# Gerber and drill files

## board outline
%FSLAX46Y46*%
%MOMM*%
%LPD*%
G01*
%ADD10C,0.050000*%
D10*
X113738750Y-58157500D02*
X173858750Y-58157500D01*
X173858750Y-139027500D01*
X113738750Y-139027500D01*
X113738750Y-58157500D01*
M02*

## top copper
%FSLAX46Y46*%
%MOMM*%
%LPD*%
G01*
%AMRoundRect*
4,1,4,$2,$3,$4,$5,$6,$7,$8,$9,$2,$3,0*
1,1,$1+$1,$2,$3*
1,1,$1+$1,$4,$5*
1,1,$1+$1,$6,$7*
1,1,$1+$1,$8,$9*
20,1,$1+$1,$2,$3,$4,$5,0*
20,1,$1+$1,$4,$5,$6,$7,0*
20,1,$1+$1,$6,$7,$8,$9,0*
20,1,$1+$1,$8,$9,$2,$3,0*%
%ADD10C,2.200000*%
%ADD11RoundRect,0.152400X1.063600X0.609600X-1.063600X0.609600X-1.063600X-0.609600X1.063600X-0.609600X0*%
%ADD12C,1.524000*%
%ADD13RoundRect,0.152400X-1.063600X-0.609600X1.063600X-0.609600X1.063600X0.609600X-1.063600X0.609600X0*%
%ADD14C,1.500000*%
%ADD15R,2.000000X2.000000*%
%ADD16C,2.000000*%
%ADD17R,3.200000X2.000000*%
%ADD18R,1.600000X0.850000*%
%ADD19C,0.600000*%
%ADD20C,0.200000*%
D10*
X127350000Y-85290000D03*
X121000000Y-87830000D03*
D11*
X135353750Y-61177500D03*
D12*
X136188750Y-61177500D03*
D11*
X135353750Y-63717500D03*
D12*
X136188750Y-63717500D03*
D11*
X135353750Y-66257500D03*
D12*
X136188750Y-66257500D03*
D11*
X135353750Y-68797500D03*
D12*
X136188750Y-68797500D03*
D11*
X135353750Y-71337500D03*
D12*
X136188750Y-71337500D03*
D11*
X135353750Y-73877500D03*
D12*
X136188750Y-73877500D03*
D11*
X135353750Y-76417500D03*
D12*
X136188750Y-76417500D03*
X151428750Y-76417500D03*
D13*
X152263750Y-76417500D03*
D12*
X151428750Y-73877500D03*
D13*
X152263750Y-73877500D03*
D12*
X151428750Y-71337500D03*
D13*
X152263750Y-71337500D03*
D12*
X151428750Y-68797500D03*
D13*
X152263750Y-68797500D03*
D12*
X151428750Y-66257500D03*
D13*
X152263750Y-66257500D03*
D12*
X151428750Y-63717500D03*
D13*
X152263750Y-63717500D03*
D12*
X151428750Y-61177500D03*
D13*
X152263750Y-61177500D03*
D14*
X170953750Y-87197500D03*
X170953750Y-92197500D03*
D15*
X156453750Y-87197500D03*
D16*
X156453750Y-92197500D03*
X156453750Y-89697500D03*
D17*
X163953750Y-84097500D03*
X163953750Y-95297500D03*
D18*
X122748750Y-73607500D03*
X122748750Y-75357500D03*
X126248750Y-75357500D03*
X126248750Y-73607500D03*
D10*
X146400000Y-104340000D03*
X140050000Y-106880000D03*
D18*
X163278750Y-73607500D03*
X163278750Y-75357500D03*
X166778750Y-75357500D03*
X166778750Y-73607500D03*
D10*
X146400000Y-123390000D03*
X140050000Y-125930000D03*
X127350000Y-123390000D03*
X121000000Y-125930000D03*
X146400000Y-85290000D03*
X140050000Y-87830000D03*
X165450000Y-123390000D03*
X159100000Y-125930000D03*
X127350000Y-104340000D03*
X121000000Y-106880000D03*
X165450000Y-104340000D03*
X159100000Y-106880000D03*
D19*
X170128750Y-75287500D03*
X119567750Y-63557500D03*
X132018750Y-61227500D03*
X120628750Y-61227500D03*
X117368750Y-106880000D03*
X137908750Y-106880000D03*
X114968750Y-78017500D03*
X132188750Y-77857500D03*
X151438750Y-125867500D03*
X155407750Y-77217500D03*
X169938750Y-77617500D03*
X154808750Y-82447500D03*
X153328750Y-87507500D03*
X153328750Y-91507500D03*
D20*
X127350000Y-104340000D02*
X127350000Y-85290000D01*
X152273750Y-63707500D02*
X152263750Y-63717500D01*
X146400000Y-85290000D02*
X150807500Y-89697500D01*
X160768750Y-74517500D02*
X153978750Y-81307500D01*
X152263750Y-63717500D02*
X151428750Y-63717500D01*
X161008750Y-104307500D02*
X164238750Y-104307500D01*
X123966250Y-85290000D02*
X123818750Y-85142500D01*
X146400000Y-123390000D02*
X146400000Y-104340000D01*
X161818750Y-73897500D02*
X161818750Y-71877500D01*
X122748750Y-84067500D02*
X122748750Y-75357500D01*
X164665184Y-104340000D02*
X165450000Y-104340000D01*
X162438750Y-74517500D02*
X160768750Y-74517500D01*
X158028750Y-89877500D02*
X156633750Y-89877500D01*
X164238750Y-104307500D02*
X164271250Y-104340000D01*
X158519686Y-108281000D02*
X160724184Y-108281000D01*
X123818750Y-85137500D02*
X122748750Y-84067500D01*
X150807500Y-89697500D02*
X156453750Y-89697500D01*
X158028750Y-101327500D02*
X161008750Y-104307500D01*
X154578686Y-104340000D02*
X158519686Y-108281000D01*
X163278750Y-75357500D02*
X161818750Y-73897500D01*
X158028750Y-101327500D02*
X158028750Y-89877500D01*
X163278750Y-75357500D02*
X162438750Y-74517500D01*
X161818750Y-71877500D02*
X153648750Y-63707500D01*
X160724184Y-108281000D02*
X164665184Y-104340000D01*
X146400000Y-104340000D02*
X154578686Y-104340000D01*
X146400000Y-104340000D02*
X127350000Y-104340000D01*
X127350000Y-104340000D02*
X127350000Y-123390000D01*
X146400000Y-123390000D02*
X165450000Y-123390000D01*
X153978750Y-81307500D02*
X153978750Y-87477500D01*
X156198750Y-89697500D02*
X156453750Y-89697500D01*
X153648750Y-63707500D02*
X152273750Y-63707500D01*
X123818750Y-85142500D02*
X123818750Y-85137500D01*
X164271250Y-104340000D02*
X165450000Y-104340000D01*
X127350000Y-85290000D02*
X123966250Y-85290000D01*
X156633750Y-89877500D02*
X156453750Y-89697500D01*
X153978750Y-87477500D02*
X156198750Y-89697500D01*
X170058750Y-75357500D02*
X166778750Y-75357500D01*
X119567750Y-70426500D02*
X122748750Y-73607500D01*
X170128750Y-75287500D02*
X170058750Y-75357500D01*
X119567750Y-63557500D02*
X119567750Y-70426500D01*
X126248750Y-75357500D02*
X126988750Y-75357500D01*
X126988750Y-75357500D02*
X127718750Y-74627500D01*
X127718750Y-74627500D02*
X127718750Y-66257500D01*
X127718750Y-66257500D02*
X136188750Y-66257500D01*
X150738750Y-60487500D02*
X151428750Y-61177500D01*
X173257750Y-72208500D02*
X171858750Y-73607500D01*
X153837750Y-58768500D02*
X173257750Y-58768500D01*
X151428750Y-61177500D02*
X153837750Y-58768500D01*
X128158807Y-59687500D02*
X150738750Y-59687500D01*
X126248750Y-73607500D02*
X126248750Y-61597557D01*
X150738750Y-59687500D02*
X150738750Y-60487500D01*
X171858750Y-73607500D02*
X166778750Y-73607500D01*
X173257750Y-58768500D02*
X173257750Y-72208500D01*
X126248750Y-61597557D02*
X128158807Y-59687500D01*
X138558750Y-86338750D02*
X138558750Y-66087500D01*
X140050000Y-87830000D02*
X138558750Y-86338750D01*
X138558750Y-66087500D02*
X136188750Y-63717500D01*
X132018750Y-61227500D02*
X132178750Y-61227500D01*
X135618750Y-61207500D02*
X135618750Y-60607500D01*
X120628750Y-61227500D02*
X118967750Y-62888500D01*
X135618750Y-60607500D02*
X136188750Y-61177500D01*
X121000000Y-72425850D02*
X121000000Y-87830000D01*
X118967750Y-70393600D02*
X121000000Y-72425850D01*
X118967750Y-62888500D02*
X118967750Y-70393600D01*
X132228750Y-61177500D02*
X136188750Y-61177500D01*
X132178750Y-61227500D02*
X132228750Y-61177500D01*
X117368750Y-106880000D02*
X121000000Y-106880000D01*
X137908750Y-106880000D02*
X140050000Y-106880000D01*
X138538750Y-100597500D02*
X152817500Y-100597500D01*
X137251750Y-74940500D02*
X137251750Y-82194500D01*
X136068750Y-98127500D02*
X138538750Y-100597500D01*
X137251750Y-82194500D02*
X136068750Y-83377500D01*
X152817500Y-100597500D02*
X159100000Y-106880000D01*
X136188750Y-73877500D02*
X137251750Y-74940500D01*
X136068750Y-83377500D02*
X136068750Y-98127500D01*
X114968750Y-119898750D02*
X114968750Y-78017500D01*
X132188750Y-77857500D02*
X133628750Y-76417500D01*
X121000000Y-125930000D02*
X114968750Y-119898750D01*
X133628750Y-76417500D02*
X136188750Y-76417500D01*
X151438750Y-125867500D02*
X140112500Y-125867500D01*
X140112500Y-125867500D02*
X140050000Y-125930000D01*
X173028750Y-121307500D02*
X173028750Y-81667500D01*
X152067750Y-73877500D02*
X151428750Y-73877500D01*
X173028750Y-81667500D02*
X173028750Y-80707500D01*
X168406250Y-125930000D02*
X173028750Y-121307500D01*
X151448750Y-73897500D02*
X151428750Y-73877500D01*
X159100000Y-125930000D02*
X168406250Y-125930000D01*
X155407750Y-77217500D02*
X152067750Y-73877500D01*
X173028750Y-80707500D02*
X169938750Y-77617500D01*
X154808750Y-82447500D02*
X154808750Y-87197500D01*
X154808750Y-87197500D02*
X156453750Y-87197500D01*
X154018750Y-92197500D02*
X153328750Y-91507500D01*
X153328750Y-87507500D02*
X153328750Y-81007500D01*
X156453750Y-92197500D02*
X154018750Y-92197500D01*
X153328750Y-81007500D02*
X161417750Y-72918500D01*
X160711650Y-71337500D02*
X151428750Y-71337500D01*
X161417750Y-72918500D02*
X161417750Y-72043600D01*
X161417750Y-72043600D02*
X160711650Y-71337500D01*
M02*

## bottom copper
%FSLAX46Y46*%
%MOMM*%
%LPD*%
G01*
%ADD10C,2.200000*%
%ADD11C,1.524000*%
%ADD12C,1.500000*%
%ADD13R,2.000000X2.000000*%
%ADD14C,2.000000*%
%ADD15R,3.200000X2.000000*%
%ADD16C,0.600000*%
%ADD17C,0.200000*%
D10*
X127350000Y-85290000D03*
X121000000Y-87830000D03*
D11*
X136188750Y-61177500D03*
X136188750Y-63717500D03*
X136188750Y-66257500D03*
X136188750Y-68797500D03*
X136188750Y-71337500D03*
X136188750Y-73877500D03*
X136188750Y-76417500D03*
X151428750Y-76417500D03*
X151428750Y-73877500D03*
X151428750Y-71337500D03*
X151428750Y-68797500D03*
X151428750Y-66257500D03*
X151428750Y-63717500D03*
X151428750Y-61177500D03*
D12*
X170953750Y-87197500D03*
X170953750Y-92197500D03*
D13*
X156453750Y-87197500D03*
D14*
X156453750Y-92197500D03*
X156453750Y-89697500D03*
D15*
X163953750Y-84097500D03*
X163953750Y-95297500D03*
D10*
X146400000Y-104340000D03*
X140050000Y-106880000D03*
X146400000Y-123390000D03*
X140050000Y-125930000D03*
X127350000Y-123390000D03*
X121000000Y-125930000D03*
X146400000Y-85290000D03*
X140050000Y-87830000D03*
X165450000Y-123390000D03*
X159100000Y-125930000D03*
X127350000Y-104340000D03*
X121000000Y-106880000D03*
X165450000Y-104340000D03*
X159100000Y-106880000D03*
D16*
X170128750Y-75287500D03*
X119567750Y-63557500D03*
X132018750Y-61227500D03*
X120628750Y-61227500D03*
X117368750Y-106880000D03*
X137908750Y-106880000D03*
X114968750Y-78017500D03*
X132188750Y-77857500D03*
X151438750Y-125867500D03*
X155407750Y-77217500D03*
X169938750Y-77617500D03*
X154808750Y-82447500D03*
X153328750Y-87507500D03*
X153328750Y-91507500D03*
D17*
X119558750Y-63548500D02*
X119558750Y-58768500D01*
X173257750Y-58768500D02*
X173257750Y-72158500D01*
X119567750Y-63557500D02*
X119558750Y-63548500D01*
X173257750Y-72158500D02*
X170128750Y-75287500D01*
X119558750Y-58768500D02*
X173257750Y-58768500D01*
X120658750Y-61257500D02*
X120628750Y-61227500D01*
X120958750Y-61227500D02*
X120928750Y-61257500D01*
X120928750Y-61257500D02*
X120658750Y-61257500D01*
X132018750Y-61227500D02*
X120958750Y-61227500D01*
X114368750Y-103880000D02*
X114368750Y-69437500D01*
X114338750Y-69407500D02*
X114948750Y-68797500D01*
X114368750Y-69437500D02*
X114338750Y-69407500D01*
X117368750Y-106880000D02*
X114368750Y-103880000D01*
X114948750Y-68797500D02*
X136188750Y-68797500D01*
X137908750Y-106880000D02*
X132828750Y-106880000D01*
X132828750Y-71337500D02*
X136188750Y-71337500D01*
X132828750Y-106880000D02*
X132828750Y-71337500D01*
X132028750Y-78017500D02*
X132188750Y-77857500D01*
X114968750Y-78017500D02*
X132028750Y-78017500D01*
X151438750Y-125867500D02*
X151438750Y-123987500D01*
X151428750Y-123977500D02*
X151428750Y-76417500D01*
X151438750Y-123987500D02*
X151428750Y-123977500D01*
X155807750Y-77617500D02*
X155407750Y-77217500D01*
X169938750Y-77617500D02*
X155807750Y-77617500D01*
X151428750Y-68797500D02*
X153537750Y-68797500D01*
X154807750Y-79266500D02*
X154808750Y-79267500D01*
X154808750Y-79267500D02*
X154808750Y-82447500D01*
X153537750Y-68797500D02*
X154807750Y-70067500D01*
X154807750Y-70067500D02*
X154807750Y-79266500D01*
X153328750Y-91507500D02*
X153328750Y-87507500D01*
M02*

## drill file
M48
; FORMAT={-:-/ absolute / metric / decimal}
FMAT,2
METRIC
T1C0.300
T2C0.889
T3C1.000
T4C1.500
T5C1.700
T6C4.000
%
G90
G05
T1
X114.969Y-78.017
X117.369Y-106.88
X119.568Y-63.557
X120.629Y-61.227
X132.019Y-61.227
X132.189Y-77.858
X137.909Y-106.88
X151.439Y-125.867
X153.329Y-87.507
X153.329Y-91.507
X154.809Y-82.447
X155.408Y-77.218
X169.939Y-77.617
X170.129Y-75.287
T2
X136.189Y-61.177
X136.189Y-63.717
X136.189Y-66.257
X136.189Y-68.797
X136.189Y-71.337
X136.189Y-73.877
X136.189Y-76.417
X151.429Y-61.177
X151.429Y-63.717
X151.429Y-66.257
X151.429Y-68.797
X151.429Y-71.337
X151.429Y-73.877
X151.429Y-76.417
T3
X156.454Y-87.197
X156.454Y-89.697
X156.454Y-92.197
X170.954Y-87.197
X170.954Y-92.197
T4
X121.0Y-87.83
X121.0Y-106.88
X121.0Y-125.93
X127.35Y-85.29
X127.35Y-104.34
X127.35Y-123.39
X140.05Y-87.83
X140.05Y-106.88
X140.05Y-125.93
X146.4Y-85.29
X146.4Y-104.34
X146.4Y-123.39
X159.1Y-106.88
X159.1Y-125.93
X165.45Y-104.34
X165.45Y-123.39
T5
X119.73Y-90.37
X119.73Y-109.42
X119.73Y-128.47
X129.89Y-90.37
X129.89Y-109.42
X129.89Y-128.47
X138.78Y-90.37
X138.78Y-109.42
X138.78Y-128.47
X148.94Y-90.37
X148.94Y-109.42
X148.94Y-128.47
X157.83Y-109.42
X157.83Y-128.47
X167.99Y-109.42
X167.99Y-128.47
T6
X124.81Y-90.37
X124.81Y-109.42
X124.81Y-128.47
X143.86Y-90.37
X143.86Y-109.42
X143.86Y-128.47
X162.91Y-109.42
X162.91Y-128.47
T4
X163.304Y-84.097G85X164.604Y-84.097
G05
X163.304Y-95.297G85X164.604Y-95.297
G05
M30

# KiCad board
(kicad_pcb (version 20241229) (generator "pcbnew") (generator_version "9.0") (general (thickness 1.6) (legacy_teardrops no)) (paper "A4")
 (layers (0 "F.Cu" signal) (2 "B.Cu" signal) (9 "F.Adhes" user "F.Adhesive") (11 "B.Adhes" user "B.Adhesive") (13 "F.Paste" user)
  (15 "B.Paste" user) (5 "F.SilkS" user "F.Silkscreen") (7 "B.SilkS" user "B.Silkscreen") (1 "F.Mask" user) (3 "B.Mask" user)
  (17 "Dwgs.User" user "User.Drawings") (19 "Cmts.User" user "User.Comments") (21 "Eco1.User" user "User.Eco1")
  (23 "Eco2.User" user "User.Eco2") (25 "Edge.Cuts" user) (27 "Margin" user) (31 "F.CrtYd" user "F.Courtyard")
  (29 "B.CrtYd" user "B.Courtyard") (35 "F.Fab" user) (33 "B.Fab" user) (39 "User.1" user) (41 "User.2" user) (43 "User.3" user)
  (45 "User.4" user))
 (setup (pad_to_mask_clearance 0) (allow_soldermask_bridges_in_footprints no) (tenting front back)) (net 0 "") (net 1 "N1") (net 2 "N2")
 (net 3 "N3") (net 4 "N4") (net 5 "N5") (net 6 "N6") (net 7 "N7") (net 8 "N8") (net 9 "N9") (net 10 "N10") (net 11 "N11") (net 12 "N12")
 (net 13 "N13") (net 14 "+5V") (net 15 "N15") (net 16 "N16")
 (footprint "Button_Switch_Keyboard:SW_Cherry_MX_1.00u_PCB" (layer "F.Cu") (at 127.35 85.29)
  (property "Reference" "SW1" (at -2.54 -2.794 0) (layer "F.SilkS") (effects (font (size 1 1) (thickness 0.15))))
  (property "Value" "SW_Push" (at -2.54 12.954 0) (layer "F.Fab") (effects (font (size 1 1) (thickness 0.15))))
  (pad "" np_thru_hole circle (at -7.62 5.08) (size 1.7 1.7) (drill 1.7) (layers "*.Cu" "*.Mask"))
  (pad "" np_thru_hole circle (at -2.54 5.08) (size 4 4) (drill 4) (layers "*.Cu" "*.Mask"))
  (pad "" np_thru_hole circle (at 2.54 5.08) (size 1.7 1.7) (drill 1.7) (layers "*.Cu" "*.Mask"))
  (pad "1" thru_hole circle (at 0 0) (size 2.2 2.2) (drill 1.5) (layers "*.Cu" "*.Mask") (remove_unused_layers no) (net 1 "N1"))
  (pad "2" thru_hole circle (at -6.35 2.54) (size 2.2 2.2) (drill 1.5) (layers "*.Cu" "*.Mask") (remove_unused_layers no) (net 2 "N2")))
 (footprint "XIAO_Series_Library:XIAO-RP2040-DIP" (layer "F.Cu") (at 143.80875 68.7975)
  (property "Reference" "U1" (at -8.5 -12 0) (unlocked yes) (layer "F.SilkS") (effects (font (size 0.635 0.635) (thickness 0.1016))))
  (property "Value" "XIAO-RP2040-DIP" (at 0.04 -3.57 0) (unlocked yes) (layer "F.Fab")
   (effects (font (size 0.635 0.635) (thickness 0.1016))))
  (pad "1" smd roundrect (at -8.455 -7.62 180) (size 2.432 1.524) (layers "F.Cu" "F.Mask") (roundrect_rratio 0.1) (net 2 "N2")
   (thermal_bridge_angle 45))
  (pad "1" thru_hole circle (at -7.62 -7.62 180) (size 1.524 1.524) (drill 0.889) (layers "*.Cu" "*.Mask") (remove_unused_layers no)
   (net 2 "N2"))
  (pad "2" smd roundrect (at -8.455 -5.08 180) (size 2.432 1.524) (layers "F.Cu" "F.Mask") (roundrect_rratio 0.1) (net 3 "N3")
   (thermal_bridge_angle 45))
  (pad "2" thru_hole circle (at -7.62 -5.08 180) (size 1.524 1.524) (drill 0.889) (layers "*.Cu" "*.Mask") (remove_unused_layers no)
   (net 3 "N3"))
  (pad "3" smd roundrect (at -8.455 -2.54 180) (size 2.432 1.524) (layers "F.Cu" "F.Mask") (roundrect_rratio 0.1) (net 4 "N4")
   (thermal_bridge_angle 45))
  (pad "3" thru_hole circle (at -7.62 -2.54 180) (size 1.524 1.524) (drill 0.889) (layers "*.Cu" "*.Mask") (remove_unused_layers no)
   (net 4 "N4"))
  (pad "4" smd roundrect (at -8.455 0 180) (size 2.432 1.524) (layers "F.Cu" "F.Mask") (roundrect_rratio 0.1) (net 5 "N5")
   (thermal_bridge_angle 45))
  (pad "4" thru_hole circle (at -7.62 0 180) (size 1.524 1.524) (drill 0.889) (layers "*.Cu" "*.Mask") (remove_unused_layers no)
   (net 5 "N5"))
  (pad "5" smd roundrect (at -8.455 2.54 180) (size 2.432 1.524) (layers "F.Cu" "F.Mask") (roundrect_rratio 0.1) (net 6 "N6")
   (thermal_bridge_angle 45))
  (pad "5" thru_hole circle (at -7.62 2.54 180) (size 1.524 1.524) (drill 0.889) (layers "*.Cu" "*.Mask") (remove_unused_layers no)
   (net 6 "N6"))
  (pad "6" smd roundrect (at -8.455 5.08 180) (size 2.432 1.524) (layers "F.Cu" "F.Mask") (roundrect_rratio 0.1) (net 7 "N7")
   (thermal_bridge_angle 45))
  (pad "6" thru_hole circle (at -7.62 5.08 180) (size 1.524 1.524) (drill 0.889) (layers "*.Cu" "*.Mask") (remove_unused_layers no)
   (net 7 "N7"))
  (pad "7" smd roundrect (at -8.455 7.62 180) (size 2.432 1.524) (layers "F.Cu" "F.Mask") (roundrect_rratio 0.1) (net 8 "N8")
   (thermal_bridge_angle 45))
  (pad "7" thru_hole circle (at -7.62 7.62 180) (size 1.524 1.524) (drill 0.889) (layers "*.Cu" "*.Mask") (remove_unused_layers no)
   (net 8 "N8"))
  (pad "8" thru_hole circle (at 7.62 7.62) (size 1.524 1.524) (drill 0.889) (layers "*.Cu" "*.Mask") (remove_unused_layers no) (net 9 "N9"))
  (pad "8" smd roundrect (at 8.455 7.62) (size 2.432 1.524) (layers "F.Cu" "F.Mask") (roundrect_rratio 0.1) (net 9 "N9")
   (thermal_bridge_angle 45))
  (pad "9" thru_hole circle (at 7.62 5.08) (size 1.524 1.524) (drill 0.889) (layers "*.Cu" "*.Mask") (remove_unused_layers no)
   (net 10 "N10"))
  (pad "9" smd roundrect (at 8.455 5.08) (size 2.432 1.524) (layers "F.Cu" "F.Mask") (roundrect_rratio 0.1) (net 10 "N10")
   (thermal_bridge_angle 45))
  (pad "10" thru_hole circle (at 7.62 2.54) (size 1.524 1.524) (drill 0.889) (layers "*.Cu" "*.Mask") (remove_unused_layers no)
   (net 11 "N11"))
  (pad "10" smd roundrect (at 8.455 2.54) (size 2.432 1.524) (layers "F.Cu" "F.Mask") (roundrect_rratio 0.1) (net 11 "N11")
   (thermal_bridge_angle 45))
  (pad "11" thru_hole circle (at 7.62 0) (size 1.524 1.524) (drill 0.889) (layers "*.Cu" "*.Mask") (remove_unused_layers no) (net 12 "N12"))
  (pad "11" smd roundrect (at 8.455 0) (size 2.432 1.524) (layers "F.Cu" "F.Mask") (roundrect_rratio 0.1) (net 12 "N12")
   (thermal_bridge_angle 45))
  (pad "12" thru_hole circle (at 7.62 -2.54) (size 1.524 1.524) (drill 0.889) (layers "*.Cu" "*.Mask") (remove_unused_layers no)
   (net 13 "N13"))
  (pad "12" smd roundrect (at 8.455 -2.54) (size 2.432 1.524) (layers "F.Cu" "F.Mask") (roundrect_rratio 0.1) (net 13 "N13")
   (thermal_bridge_angle 45))
  (pad "13" thru_hole circle (at 7.62 -5.08) (size 1.524 1.524) (drill 0.889) (layers "*.Cu" "*.Mask") (remove_unused_layers no)
   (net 1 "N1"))
  (pad "13" smd roundrect (at 8.455 -5.08) (size 2.432 1.524) (layers "F.Cu" "F.Mask") (roundrect_rratio 0.1) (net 1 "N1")
   (thermal_bridge_angle 45))
  (pad "14" thru_hole circle (at 7.62 -7.62) (size 1.524 1.524) (drill 0.889) (layers "*.Cu" "*.Mask") (remove_unused_layers no)
   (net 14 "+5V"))
  (pad "14" smd roundrect (at 8.455 -7.62) (size 2.432 1.524) (layers "F.Cu" "F.Mask") (roundrect_rratio 0.1) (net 14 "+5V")
   (thermal_bridge_angle 45)))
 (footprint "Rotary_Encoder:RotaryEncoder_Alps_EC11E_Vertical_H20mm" (layer "F.Cu") (at 156.45375 87.1975)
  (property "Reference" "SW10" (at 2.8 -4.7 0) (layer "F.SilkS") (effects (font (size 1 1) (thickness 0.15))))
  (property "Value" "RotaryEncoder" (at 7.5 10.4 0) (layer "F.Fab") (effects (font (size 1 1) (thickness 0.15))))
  (pad "" thru_hole circle (at 14.5 0) (size 1.5 1.5) (drill 1) (layers "*.Cu" "*.Mask") (remove_unused_layers no))
  (pad "" thru_hole circle (at 14.5 5) (size 1.5 1.5) (drill 1) (layers "*.Cu" "*.Mask") (remove_unused_layers no))
  (pad "A" thru_hole rect (at 0 0) (size 2 2) (drill 1) (layers "*.Cu" "*.Mask") (remove_unused_layers no) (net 12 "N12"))
  (pad "B" thru_hole circle (at 0 5) (size 2 2) (drill 1) (layers "*.Cu" "*.Mask") (remove_unused_layers no) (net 11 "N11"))
  (pad "C" thru_hole circle (at 0 2.5) (size 2 2) (drill 1) (layers "*.Cu" "*.Mask") (remove_unused_layers no) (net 1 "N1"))
  (pad "MP" thru_hole rect (at 7.5 -3.1) (size 3.2 2) (drill oval 2.8 1.5) (layers "*.Cu" "*.Mask") (remove_unused_layers no))
  (pad "MP" thru_hole rect (at 7.5 8.1) (size 3.2 2) (drill oval 2.8 1.5) (layers "*.Cu" "*.Mask") (remove_unused_layers no)))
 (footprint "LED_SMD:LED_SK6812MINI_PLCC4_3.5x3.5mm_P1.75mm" (layer "F.Cu") (at 124.49875 74.4825)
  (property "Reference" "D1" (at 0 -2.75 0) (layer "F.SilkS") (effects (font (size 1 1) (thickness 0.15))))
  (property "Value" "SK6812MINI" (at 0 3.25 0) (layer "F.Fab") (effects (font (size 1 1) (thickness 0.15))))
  (pad "1" smd rect (at -1.75 -0.875) (size 1.6 0.85) (layers "F.Cu" "F.Mask" "F.Paste") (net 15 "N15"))
  (pad "2" smd rect (at -1.75 0.875) (size 1.6 0.85) (layers "F.Cu" "F.Mask" "F.Paste") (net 1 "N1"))
  (pad "3" smd rect (at 1.75 0.875) (size 1.6 0.85) (layers "F.Cu" "F.Mask" "F.Paste") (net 4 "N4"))
  (pad "4" smd rect (at 1.75 -0.875) (size 1.6 0.85) (layers "F.Cu" "F.Mask" "F.Paste") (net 14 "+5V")))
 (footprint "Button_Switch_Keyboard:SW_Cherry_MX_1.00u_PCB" (layer "F.Cu") (at 146.4 104.34)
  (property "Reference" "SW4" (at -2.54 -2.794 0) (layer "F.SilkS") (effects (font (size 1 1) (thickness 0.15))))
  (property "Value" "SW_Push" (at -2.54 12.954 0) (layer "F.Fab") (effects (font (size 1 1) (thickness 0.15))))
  (pad "" np_thru_hole circle (at -7.62 5.08) (size 1.7 1.7) (drill 1.7) (layers "*.Cu" "*.Mask"))
  (pad "" np_thru_hole circle (at -2.54 5.08) (size 4 4) (drill 4) (layers "*.Cu" "*.Mask"))
  (pad "" np_thru_hole circle (at 2.54 5.08) (size 1.7 1.7) (drill 1.7) (layers "*.Cu" "*.Mask"))
  (pad "1" thru_hole circle (at 0 0) (size 2.2 2.2) (drill 1.5) (layers "*.Cu" "*.Mask") (remove_unused_layers no) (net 1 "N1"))
  (pad "2" thru_hole circle (at -6.35 2.54) (size 2.2 2.2) (drill 1.5) (layers "*.Cu" "*.Mask") (remove_unused_layers no) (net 6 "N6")))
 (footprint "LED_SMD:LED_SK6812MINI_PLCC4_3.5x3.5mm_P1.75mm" (layer "F.Cu") (at 165.02875 74.4825)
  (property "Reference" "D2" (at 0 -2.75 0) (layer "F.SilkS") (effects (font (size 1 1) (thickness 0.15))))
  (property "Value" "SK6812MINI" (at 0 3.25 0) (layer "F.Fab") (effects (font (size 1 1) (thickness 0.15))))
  (pad "1" smd rect (at -1.75 -0.875) (size 1.6 0.85) (layers "F.Cu" "F.Mask" "F.Paste") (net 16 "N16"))
  (pad "2" smd rect (at -1.75 0.875) (size 1.6 0.85) (layers "F.Cu" "F.Mask" "F.Paste") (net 1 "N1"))
  (pad "3" smd rect (at 1.75 0.875) (size 1.6 0.85) (layers "F.Cu" "F.Mask" "F.Paste") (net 15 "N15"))
  (pad "4" smd rect (at 1.75 -0.875) (size 1.6 0.85) (layers "F.Cu" "F.Mask" "F.Paste") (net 14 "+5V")))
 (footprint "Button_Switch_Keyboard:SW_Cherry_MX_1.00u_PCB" (layer "F.Cu") (at 146.4 123.39)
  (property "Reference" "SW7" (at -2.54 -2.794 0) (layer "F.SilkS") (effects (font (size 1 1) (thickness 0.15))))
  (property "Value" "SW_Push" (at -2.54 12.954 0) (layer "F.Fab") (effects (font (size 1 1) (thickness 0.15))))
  (pad "" np_thru_hole circle (at -7.62 5.08) (size 1.7 1.7) (drill 1.7) (layers "*.Cu" "*.Mask"))
  (pad "" np_thru_hole circle (at -2.54 5.08) (size 4 4) (drill 4) (layers "*.Cu" "*.Mask"))
  (pad "" np_thru_hole circle (at 2.54 5.08) (size 1.7 1.7) (drill 1.7) (layers "*.Cu" "*.Mask"))
  (pad "1" thru_hole circle (at 0 0) (size 2.2 2.2) (drill 1.5) (layers "*.Cu" "*.Mask") (remove_unused_layers no) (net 1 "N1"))
  (pad "2" thru_hole circle (at -6.35 2.54) (size 2.2 2.2) (drill 1.5) (layers "*.Cu" "*.Mask") (remove_unused_layers no) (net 9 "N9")))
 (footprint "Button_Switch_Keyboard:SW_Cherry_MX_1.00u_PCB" (layer "F.Cu") (at 127.35 123.39)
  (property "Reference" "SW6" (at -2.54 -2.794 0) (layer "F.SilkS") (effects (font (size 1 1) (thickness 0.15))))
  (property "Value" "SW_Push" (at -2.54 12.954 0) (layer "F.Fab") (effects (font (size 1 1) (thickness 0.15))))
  (pad "" np_thru_hole circle (at -7.62 5.08) (size 1.7 1.7) (drill 1.7) (layers "*.Cu" "*.Mask"))
  (pad "" np_thru_hole circle (at -2.54 5.08) (size 4 4) (drill 4) (layers "*.Cu" "*.Mask"))
  (pad "" np_thru_hole circle (at 2.54 5.08) (size 1.7 1.7) (drill 1.7) (layers "*.Cu" "*.Mask"))
  (pad "1" thru_hole circle (at 0 0) (size 2.2 2.2) (drill 1.5) (layers "*.Cu" "*.Mask") (remove_unused_layers no) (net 1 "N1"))
  (pad "2" thru_hole circle (at -6.35 2.54) (size 2.2 2.2) (drill 1.5) (layers "*.Cu" "*.Mask") (remove_unused_layers no) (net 8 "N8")))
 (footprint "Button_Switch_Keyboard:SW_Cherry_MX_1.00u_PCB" (layer "F.Cu") (at 146.4 85.29)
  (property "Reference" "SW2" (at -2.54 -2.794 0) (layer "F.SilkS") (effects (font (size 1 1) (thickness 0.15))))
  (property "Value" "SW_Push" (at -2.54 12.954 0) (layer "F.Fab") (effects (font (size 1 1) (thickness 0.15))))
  (pad "" np_thru_hole circle (at -7.62 5.08) (size 1.7 1.7) (drill 1.7) (layers "*.Cu" "*.Mask"))
  (pad "" np_thru_hole circle (at -2.54 5.08) (size 4 4) (drill 4) (layers "*.Cu" "*.Mask"))
  (pad "" np_thru_hole circle (at 2.54 5.08) (size 1.7 1.7) (drill 1.7) (layers "*.Cu" "*.Mask"))
  (pad "1" thru_hole circle (at 0 0) (size 2.2 2.2) (drill 1.5) (layers "*.Cu" "*.Mask") (remove_unused_layers no) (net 1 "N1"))
  (pad "2" thru_hole circle (at -6.35 2.54) (size 2.2 2.2) (drill 1.5) (layers "*.Cu" "*.Mask") (remove_unused_layers no) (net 3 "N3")))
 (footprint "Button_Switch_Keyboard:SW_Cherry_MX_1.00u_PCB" (layer "F.Cu") (at 165.45 123.39)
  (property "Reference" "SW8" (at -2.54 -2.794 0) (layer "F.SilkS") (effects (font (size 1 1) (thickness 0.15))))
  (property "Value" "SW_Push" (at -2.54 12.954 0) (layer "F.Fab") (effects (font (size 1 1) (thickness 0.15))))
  (pad "" np_thru_hole circle (at -7.62 5.08) (size 1.7 1.7) (drill 1.7) (layers "*.Cu" "*.Mask"))
  (pad "" np_thru_hole circle (at -2.54 5.08) (size 4 4) (drill 4) (layers "*.Cu" "*.Mask"))
  (pad "" np_thru_hole circle (at 2.54 5.08) (size 1.7 1.7) (drill 1.7) (layers "*.Cu" "*.Mask"))
  (pad "1" thru_hole circle (at 0 0) (size 2.2 2.2) (drill 1.5) (layers "*.Cu" "*.Mask") (remove_unused_layers no) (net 1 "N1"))
  (pad "2" thru_hole circle (at -6.35 2.54) (size 2.2 2.2) (drill 1.5) (layers "*.Cu" "*.Mask") (remove_unused_layers no) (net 10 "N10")))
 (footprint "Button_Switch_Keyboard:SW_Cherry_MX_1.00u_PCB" (layer "F.Cu") (at 127.35 104.34)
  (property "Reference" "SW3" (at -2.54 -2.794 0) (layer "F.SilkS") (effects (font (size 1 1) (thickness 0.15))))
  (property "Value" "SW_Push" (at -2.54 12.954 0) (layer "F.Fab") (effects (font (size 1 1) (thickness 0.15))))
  (pad "" np_thru_hole circle (at -7.62 5.08) (size 1.7 1.7) (drill 1.7) (layers "*.Cu" "*.Mask"))
  (pad "" np_thru_hole circle (at -2.54 5.08) (size 4 4) (drill 4) (layers "*.Cu" "*.Mask"))
  (pad "" np_thru_hole circle (at 2.54 5.08) (size 1.7 1.7) (drill 1.7) (layers "*.Cu" "*.Mask"))
  (pad "1" thru_hole circle (at 0 0) (size 2.2 2.2) (drill 1.5) (layers "*.Cu" "*.Mask") (remove_unused_layers no) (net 1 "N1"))
  (pad "2" thru_hole circle (at -6.35 2.54) (size 2.2 2.2) (drill 1.5) (layers "*.Cu" "*.Mask") (remove_unused_layers no) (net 5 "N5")))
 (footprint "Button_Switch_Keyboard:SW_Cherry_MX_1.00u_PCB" (layer "F.Cu") (at 165.45 104.34)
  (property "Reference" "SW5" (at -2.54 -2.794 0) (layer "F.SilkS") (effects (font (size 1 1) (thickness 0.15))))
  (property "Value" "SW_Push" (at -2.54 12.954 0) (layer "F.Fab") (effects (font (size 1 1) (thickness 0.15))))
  (pad "" np_thru_hole circle (at -7.62 5.08) (size 1.7 1.7) (drill 1.7) (layers "*.Cu" "*.Mask"))
  (pad "" np_thru_hole circle (at -2.54 5.08) (size 4 4) (drill 4) (layers "*.Cu" "*.Mask"))
  (pad "" np_thru_hole circle (at 2.54 5.08) (size 1.7 1.7) (drill 1.7) (layers "*.Cu" "*.Mask"))
  (pad "1" thru_hole circle (at 0 0) (size 2.2 2.2) (drill 1.5) (layers "*.Cu" "*.Mask") (remove_unused_layers no) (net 1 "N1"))
  (pad "2" thru_hole circle (at -6.35 2.54) (size 2.2 2.2) (drill 1.5) (layers "*.Cu" "*.Mask") (remove_unused_layers no) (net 7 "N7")))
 (gr_rect (start 113.73875 58.1575) (end 173.85875 139.0275) (stroke (width 0.05) (type default)) (fill no) (layer "Edge.Cuts"))
 (segment (start 127.35 104.34) (end 127.35 85.29) (width 0.2) (layer "F.Cu") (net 1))
 (segment (start 152.27375 63.7075) (end 152.26375 63.7175) (width 0.2) (layer "F.Cu") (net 1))
 (segment (start 146.4 85.29) (end 150.8075 89.6975) (width 0.2) (layer "F.Cu") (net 1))
 (segment (start 160.76875 74.5175) (end 153.97875 81.3075) (width 0.2) (layer "F.Cu") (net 1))
 (segment (start 152.26375 63.7175) (end 151.42875 63.7175) (width 0.2) (layer "F.Cu") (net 1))
 (segment (start 161.00875 104.3075) (end 164.23875 104.3075) (width 0.2) (layer "F.Cu") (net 1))
 (segment (start 123.96625 85.29) (end 123.81875 85.1425) (width 0.2) (layer "F.Cu") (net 1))
 (segment (start 146.4 123.39) (end 146.4 104.34) (width 0.2) (layer "F.Cu") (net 1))
 (segment (start 161.81875 73.8975) (end 161.81875 71.8775) (width 0.2) (layer "F.Cu") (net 1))
 (segment (start 122.74875 84.0675) (end 122.74875 75.3575) (width 0.2) (layer "F.Cu") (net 1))
 (segment (start 164.665184 104.34) (end 165.45 104.34) (width 0.2) (layer "F.Cu") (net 1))
 (segment (start 162.43875 74.5175) (end 160.76875 74.5175) (width 0.2) (layer "F.Cu") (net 1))
 (segment (start 158.02875 89.8775) (end 156.63375 89.8775) (width 0.2) (layer "F.Cu") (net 1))
 (segment (start 164.23875 104.3075) (end 164.27125 104.34) (width 0.2) (layer "F.Cu") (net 1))
 (segment (start 158.519686 108.281) (end 160.724184 108.281) (width 0.2) (layer "F.Cu") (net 1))
 (segment (start 123.81875 85.1375) (end 122.74875 84.0675) (width 0.2) (layer "F.Cu") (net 1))
 (segment (start 150.8075 89.6975) (end 156.45375 89.6975) (width 0.2) (layer "F.Cu") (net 1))
 (segment (start 158.02875 101.3275) (end 161.00875 104.3075) (width 0.2) (layer "F.Cu") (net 1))
 (segment (start 154.578686 104.34) (end 158.519686 108.281) (width 0.2) (layer "F.Cu") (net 1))
 (segment (start 163.27875 75.3575) (end 161.81875 73.8975) (width 0.2) (layer "F.Cu") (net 1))
 (segment (start 158.02875 101.3275) (end 158.02875 89.8775) (width 0.2) (layer "F.Cu") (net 1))
 (segment (start 163.27875 75.3575) (end 162.43875 74.5175) (width 0.2) (layer "F.Cu") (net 1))
 (segment (start 161.81875 71.8775) (end 153.64875 63.7075) (width 0.2) (layer "F.Cu") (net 1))
 (segment (start 160.724184 108.281) (end 164.665184 104.34) (width 0.2) (layer "F.Cu") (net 1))
 (segment (start 146.4 104.34) (end 154.578686 104.34) (width 0.2) (layer "F.Cu") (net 1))
 (segment (start 146.4 104.34) (end 127.35 104.34) (width 0.2) (layer "F.Cu") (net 1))
 (segment (start 127.35 104.34) (end 127.35 123.39) (width 0.2) (layer "F.Cu") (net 1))
 (segment (start 146.4 123.39) (end 165.45 123.39) (width 0.2) (layer "F.Cu") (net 1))
 (segment (start 153.97875 81.3075) (end 153.97875 87.4775) (width 0.2) (layer "F.Cu") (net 1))
 (segment (start 156.19875 89.6975) (end 156.45375 89.6975) (width 0.2) (layer "F.Cu") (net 1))
 (segment (start 153.64875 63.7075) (end 152.27375 63.7075) (width 0.2) (layer "F.Cu") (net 1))
 (segment (start 123.81875 85.1425) (end 123.81875 85.1375) (width 0.2) (layer "F.Cu") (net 1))
 (segment (start 164.27125 104.34) (end 165.45 104.34) (width 0.2) (layer "F.Cu") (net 1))
 (segment (start 127.35 85.29) (end 123.96625 85.29) (width 0.2) (layer "F.Cu") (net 1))
 (segment (start 156.63375 89.8775) (end 156.45375 89.6975) (width 0.2) (layer "F.Cu") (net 1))
 (segment (start 153.97875 87.4775) (end 156.19875 89.6975) (width 0.2) (layer "F.Cu") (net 1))
 (segment (start 170.05875 75.3575) (end 166.77875 75.3575) (width 0.2) (layer "F.Cu") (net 15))
 (segment (start 119.56775 70.4265) (end 122.74875 73.6075) (width 0.2) (layer "F.Cu") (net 15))
 (segment (start 170.12875 75.2875) (end 170.05875 75.3575) (width 0.2) (layer "F.Cu") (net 15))
 (segment (start 119.56775 63.5575) (end 119.56775 70.4265) (width 0.2) (layer "F.Cu") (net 15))
 (via (at 170.12875 75.2875) (size 0.6) (drill 0.3) (layers "F.Cu" "B.Cu") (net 15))
 (via (at 119.56775 63.5575) (size 0.6) (drill 0.3) (layers "F.Cu" "B.Cu") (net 15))
 (segment (start 119.55875 63.5485) (end 119.55875 58.7685) (width 0.2) (layer "B.Cu") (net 15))
 (segment (start 173.25775 58.7685) (end 173.25775 72.1585) (width 0.2) (layer "B.Cu") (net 15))
 (segment (start 119.56775 63.5575) (end 119.55875 63.5485) (width 0.2) (layer "B.Cu") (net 15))
 (segment (start 173.25775 72.1585) (end 170.12875 75.2875) (width 0.2) (layer "B.Cu") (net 15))
 (segment (start 119.55875 58.7685) (end 173.25775 58.7685) (width 0.2) (layer "B.Cu") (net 15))
 (segment (start 126.24875 75.3575) (end 126.98875 75.3575) (width 0.2) (layer "F.Cu") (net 4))
 (segment (start 126.98875 75.3575) (end 127.71875 74.6275) (width 0.2) (layer "F.Cu") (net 4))
 (segment (start 127.71875 74.6275) (end 127.71875 66.2575) (width 0.2) (layer "F.Cu") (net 4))
 (segment (start 127.71875 66.2575) (end 136.18875 66.2575) (width 0.2) (layer "F.Cu") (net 4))
 (segment (start 150.73875 60.4875) (end 151.42875 61.1775) (width 0.2) (layer "F.Cu") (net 14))
 (segment (start 173.25775 72.2085) (end 171.85875 73.6075) (width 0.2) (layer "F.Cu") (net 14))
 (segment (start 153.83775 58.7685) (end 173.25775 58.7685) (width 0.2) (layer "F.Cu") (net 14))
 (segment (start 151.42875 61.1775) (end 153.83775 58.7685) (width 0.2) (layer "F.Cu") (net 14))
 (segment (start 128.158807 59.6875) (end 150.73875 59.6875) (width 0.2) (layer "F.Cu") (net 14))
 (segment (start 126.24875 73.6075) (end 126.24875 61.597557) (width 0.2) (layer "F.Cu") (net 14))
 (segment (start 150.73875 59.6875) (end 150.73875 60.4875) (width 0.2) (layer "F.Cu") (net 14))
 (segment (start 171.85875 73.6075) (end 166.77875 73.6075) (width 0.2) (layer "F.Cu") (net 14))
 (segment (start 173.25775 58.7685) (end 173.25775 72.2085) (width 0.2) (layer "F.Cu") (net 14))
 (segment (start 126.24875 61.597557) (end 128.158807 59.6875) (width 0.2) (layer "F.Cu") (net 14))
 (segment (start 138.55875 86.33875) (end 138.55875 66.0875) (width 0.2) (layer "F.Cu") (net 3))
 (segment (start 140.05 87.83) (end 138.55875 86.33875) (width 0.2) (layer "F.Cu") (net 3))
 (segment (start 138.55875 66.0875) (end 136.18875 63.7175) (width 0.2) (layer "F.Cu") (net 3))
 (segment (start 132.01875 61.2275) (end 132.17875 61.2275) (width 0.2) (layer "F.Cu") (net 2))
 (segment (start 135.61875 61.2075) (end 135.61875 60.6075) (width 0.2) (layer "F.Cu") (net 2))
 (segment (start 120.62875 61.2275) (end 118.96775 62.8885) (width 0.2) (layer "F.Cu") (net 2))
 (segment (start 135.61875 60.6075) (end 136.18875 61.1775) (width 0.2) (layer "F.Cu") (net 2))
 (segment (start 121 72.42585) (end 121 87.83) (width 0.2) (layer "F.Cu") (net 2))
 (segment (start 118.96775 70.3936) (end 121 72.42585) (width 0.2) (layer "F.Cu") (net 2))
 (segment (start 118.96775 62.8885) (end 118.96775 70.3936) (width 0.2) (layer "F.Cu") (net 2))
 (segment (start 132.22875 61.1775) (end 136.18875 61.1775) (width 0.2) (layer "F.Cu") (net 2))
 (segment (start 132.17875 61.2275) (end 132.22875 61.1775) (width 0.2) (layer "F.Cu") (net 2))
 (via (at 132.01875 61.2275) (size 0.6) (drill 0.3) (layers "F.Cu" "B.Cu") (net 2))
 (via (at 120.62875 61.2275) (size 0.6) (drill 0.3) (layers "F.Cu" "B.Cu") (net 2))
 (segment (start 120.65875 61.2575) (end 120.62875 61.2275) (width 0.2) (layer "B.Cu") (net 2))
 (segment (start 120.95875 61.2275) (end 120.92875 61.2575) (width 0.2) (layer "B.Cu") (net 2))
 (segment (start 120.92875 61.2575) (end 120.65875 61.2575) (width 0.2) (layer "B.Cu") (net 2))
 (segment (start 132.01875 61.2275) (end 120.95875 61.2275) (width 0.2) (layer "B.Cu") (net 2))
 (segment (start 117.36875 106.88) (end 121 106.88) (width 0.2) (layer "F.Cu") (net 5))
 (via (at 117.36875 106.88) (size 0.6) (drill 0.3) (layers "F.Cu" "B.Cu") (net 5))
 (segment (start 114.36875 103.88) (end 114.36875 69.4375) (width 0.2) (layer "B.Cu") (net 5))
 (segment (start 114.33875 69.4075) (end 114.94875 68.7975) (width 0.2) (layer "B.Cu") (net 5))
 (segment (start 114.36875 69.4375) (end 114.33875 69.4075) (width 0.2) (layer "B.Cu") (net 5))
 (segment (start 117.36875 106.88) (end 114.36875 103.88) (width 0.2) (layer "B.Cu") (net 5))
 (segment (start 114.94875 68.7975) (end 136.18875 68.7975) (width 0.2) (layer "B.Cu") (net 5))
 (segment (start 137.90875 106.88) (end 140.05 106.88) (width 0.2) (layer "F.Cu") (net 6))
 (via (at 137.90875 106.88) (size 0.6) (drill 0.3) (layers "F.Cu" "B.Cu") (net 6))
 (segment (start 137.90875 106.88) (end 132.82875 106.88) (width 0.2) (layer "B.Cu") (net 6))
 (segment (start 132.82875 71.3375) (end 136.18875 71.3375) (width 0.2) (layer "B.Cu") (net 6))
 (segment (start 132.82875 106.88) (end 132.82875 71.3375) (width 0.2) (layer "B.Cu") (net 6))
 (segment (start 138.53875 100.5975) (end 152.8175 100.5975) (width 0.2) (layer "F.Cu") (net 7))
 (segment (start 137.25175 74.9405) (end 137.25175 82.1945) (width 0.2) (layer "F.Cu") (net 7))
 (segment (start 136.06875 98.1275) (end 138.53875 100.5975) (width 0.2) (layer "F.Cu") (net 7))
 (segment (start 137.25175 82.1945) (end 136.06875 83.3775) (width 0.2) (layer "F.Cu") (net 7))
 (segment (start 152.8175 100.5975) (end 159.1 106.88) (width 0.2) (layer "F.Cu") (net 7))
 (segment (start 136.18875 73.8775) (end 137.25175 74.9405) (width 0.2) (layer "F.Cu") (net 7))
 (segment (start 136.06875 83.3775) (end 136.06875 98.1275) (width 0.2) (layer "F.Cu") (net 7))
 (segment (start 114.96875 119.89875) (end 114.96875 78.0175) (width 0.2) (layer "F.Cu") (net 8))
 (segment (start 132.18875 77.8575) (end 133.62875 76.4175) (width 0.2) (layer "F.Cu") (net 8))
 (segment (start 121 125.93) (end 114.96875 119.89875) (width 0.2) (layer "F.Cu") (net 8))
 (segment (start 133.62875 76.4175) (end 136.18875 76.4175) (width 0.2) (layer "F.Cu") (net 8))
 (via (at 114.96875 78.0175) (size 0.6) (drill 0.3) (layers "F.Cu" "B.Cu") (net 8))
 (via (at 132.18875 77.8575) (size 0.6) (drill 0.3) (layers "F.Cu" "B.Cu") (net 8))
 (segment (start 132.02875 78.0175) (end 132.18875 77.8575) (width 0.2) (layer "B.Cu") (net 8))
 (segment (start 114.96875 78.0175) (end 132.02875 78.0175) (width 0.2) (layer "B.Cu") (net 8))
 (segment (start 151.43875 125.8675) (end 140.1125 125.8675) (width 0.2) (layer "F.Cu") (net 9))
 (segment (start 140.1125 125.8675) (end 140.05 125.93) (width 0.2) (layer "F.Cu") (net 9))
 (via (at 151.43875 125.8675) (size 0.6) (drill 0.3) (layers "F.Cu" "B.Cu") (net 9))
 (segment (start 151.43875 125.8675) (end 151.43875 123.9875) (width 0.2) (layer "B.Cu") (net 9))
 (segment (start 151.42875 123.9775) (end 151.42875 76.4175) (width 0.2) (layer "B.Cu") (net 9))
 (segment (start 151.43875 123.9875) (end 151.42875 123.9775) (width 0.2) (layer "B.Cu") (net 9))
 (segment (start 173.02875 121.3075) (end 173.02875 81.6675) (width 0.2) (layer "F.Cu") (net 10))
 (segment (start 152.06775 73.8775) (end 151.42875 73.8775) (width 0.2) (layer "F.Cu") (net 10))
 (segment (start 173.02875 81.6675) (end 173.02875 80.7075) (width 0.2) (layer "F.Cu") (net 10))
 (segment (start 168.40625 125.93) (end 173.02875 121.3075) (width 0.2) (layer "F.Cu") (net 10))
 (segment (start 151.44875 73.8975) (end 151.42875 73.8775) (width 0.2) (layer "F.Cu") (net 10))
 (segment (start 159.1 125.93) (end 168.40625 125.93) (width 0.2) (layer "F.Cu") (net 10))
 (segment (start 155.40775 77.2175) (end 152.06775 73.8775) (width 0.2) (layer "F.Cu") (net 10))
 (segment (start 173.02875 80.7075) (end 169.93875 77.6175) (width 0.2) (layer "F.Cu") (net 10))
 (via (at 155.40775 77.2175) (size 0.6) (drill 0.3) (layers "F.Cu" "B.Cu") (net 10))
 (via (at 169.93875 77.6175) (size 0.6) (drill 0.3) (layers "F.Cu" "B.Cu") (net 10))
 (segment (start 155.80775 77.6175) (end 155.40775 77.2175) (width 0.2) (layer "B.Cu") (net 10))
 (segment (start 169.93875 77.6175) (end 155.80775 77.6175) (width 0.2) (layer "B.Cu") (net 10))
 (segment (start 154.80875 82.4475) (end 154.80875 87.1975) (width 0.2) (layer "F.Cu") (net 12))
 (segment (start 154.80875 87.1975) (end 156.45375 87.1975) (width 0.2) (layer "F.Cu") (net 12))
 (via (at 154.80875 82.4475) (size 0.6) (drill 0.3) (layers "F.Cu" "B.Cu") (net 12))
 (segment (start 151.42875 68.7975) (end 153.53775 68.7975) (width 0.2) (layer "B.Cu") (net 12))
 (segment (start 154.80775 79.2665) (end 154.80875 79.2675) (width 0.2) (layer "B.Cu") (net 12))
 (segment (start 154.80875 79.2675) (end 154.80875 82.4475) (width 0.2) (layer "B.Cu") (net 12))
 (segment (start 153.53775 68.7975) (end 154.80775 70.0675) (width 0.2) (layer "B.Cu") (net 12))
 (segment (start 154.80775 70.0675) (end 154.80775 79.2665) (width 0.2) (layer "B.Cu") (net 12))
 (segment (start 154.01875 92.1975) (end 153.32875 91.5075) (width 0.2) (layer "F.Cu") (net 11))
 (segment (start 153.32875 87.5075) (end 153.32875 81.0075) (width 0.2) (layer "F.Cu") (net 11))
 (segment (start 156.45375 92.1975) (end 154.01875 92.1975) (width 0.2) (layer "F.Cu") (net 11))
 (segment (start 153.32875 81.0075) (end 161.41775 72.9185) (width 0.2) (layer "F.Cu") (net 11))
 (segment (start 160.71165 71.3375) (end 151.42875 71.3375) (width 0.2) (layer "F.Cu") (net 11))
 (segment (start 161.41775 72.9185) (end 161.41775 72.0436) (width 0.2) (layer "F.Cu") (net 11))
 (segment (start 161.41775 72.0436) (end 160.71165 71.3375) (width 0.2) (layer "F.Cu") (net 11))
 (via (at 153.32875 87.5075) (size 0.6) (drill 0.3) (layers "F.Cu" "B.Cu") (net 11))
 (via (at 153.32875 91.5075) (size 0.6) (drill 0.3) (layers "F.Cu" "B.Cu") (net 11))
 (segment (start 153.32875 91.5075) (end 153.32875 87.5075) (width 0.2) (layer "B.Cu") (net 11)))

